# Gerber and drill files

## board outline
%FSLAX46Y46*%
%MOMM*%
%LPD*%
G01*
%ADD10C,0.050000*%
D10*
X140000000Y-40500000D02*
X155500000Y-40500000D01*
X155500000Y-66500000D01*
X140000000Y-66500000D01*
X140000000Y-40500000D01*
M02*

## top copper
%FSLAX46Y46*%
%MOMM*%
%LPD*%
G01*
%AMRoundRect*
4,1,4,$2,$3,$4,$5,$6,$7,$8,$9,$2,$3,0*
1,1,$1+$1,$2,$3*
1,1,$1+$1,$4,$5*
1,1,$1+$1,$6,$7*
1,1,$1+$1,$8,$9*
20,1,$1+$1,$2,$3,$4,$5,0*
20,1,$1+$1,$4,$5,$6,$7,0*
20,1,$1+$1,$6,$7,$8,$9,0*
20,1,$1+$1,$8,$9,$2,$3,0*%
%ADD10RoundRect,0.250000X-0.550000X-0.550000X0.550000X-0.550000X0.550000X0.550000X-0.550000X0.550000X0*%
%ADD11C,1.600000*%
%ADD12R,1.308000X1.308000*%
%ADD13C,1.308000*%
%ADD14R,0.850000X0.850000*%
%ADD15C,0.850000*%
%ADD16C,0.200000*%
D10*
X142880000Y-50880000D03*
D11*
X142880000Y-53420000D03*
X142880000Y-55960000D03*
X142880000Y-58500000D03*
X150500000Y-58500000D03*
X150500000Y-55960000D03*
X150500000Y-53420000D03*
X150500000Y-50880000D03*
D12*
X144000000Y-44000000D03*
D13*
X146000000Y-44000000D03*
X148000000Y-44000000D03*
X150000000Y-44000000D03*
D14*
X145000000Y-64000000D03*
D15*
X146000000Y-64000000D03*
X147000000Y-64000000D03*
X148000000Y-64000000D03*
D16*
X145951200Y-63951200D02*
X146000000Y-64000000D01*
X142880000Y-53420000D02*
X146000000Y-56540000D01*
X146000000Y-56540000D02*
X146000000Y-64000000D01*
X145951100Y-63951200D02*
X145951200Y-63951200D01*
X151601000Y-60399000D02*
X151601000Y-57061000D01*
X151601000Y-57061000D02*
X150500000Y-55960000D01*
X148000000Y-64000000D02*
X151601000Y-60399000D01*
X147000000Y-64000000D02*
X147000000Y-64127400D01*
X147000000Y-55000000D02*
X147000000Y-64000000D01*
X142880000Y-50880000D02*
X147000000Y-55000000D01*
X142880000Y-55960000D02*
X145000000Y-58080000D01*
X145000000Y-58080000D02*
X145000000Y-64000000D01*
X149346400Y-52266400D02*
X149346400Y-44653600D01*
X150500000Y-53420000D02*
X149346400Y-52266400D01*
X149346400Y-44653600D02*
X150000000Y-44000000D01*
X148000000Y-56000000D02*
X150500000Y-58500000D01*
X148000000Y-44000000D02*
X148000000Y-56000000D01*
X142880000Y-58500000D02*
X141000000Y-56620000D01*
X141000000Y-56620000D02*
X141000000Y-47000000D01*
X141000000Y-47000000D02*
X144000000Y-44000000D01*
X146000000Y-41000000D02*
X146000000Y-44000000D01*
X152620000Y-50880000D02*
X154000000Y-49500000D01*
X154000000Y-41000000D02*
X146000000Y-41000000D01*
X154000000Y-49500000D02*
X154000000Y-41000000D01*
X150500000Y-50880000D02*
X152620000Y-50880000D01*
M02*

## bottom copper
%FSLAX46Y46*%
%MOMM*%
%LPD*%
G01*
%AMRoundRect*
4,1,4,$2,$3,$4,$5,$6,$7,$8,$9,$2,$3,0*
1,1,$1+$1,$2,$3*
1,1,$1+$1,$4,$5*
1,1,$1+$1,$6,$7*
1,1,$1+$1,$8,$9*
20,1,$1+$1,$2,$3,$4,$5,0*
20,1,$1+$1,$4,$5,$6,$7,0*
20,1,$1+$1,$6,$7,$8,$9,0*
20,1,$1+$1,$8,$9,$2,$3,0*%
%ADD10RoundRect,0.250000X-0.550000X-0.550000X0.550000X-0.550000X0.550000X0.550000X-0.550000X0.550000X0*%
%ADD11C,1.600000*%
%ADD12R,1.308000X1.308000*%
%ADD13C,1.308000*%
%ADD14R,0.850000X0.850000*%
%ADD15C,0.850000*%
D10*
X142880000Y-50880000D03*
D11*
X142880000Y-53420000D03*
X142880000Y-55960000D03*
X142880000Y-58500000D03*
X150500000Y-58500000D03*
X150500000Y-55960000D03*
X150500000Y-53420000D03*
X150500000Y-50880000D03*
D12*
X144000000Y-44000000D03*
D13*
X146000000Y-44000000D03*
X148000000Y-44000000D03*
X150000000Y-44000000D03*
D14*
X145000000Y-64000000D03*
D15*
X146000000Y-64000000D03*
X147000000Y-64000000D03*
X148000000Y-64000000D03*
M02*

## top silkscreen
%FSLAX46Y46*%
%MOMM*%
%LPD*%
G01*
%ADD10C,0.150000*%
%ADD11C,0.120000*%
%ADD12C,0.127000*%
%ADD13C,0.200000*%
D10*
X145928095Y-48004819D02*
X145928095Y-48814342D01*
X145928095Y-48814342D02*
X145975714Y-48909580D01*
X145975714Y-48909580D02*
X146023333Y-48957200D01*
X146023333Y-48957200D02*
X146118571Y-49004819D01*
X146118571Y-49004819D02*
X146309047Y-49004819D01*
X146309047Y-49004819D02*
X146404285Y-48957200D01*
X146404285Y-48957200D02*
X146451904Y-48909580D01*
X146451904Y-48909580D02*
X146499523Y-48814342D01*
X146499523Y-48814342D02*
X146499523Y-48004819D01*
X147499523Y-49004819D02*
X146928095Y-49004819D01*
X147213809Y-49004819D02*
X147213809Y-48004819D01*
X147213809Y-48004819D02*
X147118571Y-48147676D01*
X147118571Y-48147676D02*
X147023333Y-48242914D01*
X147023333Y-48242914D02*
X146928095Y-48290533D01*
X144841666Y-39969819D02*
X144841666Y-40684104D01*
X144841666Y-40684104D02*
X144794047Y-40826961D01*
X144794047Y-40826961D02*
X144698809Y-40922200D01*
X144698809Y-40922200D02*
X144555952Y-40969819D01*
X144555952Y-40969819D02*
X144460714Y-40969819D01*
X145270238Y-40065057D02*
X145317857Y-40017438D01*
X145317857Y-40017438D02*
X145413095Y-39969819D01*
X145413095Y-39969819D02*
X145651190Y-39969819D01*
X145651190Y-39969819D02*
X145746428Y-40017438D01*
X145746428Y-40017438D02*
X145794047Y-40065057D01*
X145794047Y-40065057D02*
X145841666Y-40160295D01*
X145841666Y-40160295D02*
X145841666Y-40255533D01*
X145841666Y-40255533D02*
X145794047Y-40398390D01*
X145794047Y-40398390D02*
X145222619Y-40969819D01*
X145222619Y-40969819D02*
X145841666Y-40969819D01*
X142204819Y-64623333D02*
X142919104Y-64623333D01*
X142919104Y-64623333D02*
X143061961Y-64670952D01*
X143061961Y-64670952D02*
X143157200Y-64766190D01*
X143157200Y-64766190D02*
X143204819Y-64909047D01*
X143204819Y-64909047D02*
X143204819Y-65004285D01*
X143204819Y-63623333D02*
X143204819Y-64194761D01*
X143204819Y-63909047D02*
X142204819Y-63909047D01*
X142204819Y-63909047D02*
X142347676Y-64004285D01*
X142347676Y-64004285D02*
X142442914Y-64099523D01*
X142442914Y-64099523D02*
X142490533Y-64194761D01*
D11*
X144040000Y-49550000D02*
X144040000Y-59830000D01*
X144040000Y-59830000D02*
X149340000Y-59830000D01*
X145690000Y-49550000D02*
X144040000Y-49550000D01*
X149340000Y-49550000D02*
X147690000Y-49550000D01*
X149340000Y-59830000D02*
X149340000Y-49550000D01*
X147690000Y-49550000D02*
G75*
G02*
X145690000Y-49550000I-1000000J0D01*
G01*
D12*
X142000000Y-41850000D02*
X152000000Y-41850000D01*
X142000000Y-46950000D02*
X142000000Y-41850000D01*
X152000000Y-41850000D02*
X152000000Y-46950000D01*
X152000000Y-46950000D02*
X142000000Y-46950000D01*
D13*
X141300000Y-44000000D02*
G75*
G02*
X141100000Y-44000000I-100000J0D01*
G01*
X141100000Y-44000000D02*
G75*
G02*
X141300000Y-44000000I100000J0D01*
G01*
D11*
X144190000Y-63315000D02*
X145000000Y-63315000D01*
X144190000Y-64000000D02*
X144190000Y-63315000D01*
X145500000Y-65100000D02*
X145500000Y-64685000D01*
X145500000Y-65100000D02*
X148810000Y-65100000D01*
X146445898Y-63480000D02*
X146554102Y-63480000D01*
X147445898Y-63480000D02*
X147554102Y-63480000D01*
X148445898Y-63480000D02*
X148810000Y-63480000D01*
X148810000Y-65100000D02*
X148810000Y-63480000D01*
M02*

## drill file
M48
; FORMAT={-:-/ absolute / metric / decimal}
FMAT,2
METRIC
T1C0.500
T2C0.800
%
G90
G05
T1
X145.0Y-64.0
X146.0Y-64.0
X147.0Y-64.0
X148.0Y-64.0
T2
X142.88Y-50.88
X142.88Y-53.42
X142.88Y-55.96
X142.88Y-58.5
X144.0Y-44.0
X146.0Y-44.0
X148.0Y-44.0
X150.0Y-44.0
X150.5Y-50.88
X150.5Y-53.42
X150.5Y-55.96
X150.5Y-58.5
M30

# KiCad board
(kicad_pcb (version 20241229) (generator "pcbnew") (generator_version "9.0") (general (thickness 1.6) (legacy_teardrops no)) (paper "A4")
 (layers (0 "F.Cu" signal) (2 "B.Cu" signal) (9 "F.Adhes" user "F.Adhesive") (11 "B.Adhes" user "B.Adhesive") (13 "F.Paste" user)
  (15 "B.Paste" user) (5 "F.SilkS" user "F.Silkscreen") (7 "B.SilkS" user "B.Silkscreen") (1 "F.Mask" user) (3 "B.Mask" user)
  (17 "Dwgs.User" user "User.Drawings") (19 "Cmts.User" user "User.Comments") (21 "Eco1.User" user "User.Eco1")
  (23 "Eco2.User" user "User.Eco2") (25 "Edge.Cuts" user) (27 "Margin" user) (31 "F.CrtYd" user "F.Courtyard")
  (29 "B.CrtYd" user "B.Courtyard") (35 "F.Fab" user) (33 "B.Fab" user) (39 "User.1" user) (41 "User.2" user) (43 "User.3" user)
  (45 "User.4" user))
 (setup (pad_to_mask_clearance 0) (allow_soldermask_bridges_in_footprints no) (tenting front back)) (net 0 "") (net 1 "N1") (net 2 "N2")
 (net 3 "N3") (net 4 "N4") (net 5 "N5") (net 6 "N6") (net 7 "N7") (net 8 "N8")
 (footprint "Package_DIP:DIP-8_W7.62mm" (layer "F.Cu") (at 142.88 50.88)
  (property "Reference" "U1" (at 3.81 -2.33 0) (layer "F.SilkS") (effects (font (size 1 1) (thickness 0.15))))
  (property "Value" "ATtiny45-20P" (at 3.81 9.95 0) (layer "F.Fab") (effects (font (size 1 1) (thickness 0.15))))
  (fp_line (start 1.16 -1.33) (end 1.16 8.95) (stroke (width 0.12) (type solid)) (layer "F.SilkS"))
  (fp_line (start 1.16 8.95) (end 6.46 8.95) (stroke (width 0.12) (type solid)) (layer "F.SilkS"))
  (fp_line (start 2.81 -1.33) (end 1.16 -1.33) (stroke (width 0.12) (type solid)) (layer "F.SilkS"))
  (fp_line (start 6.46 -1.33) (end 4.81 -1.33) (stroke (width 0.12) (type solid)) (layer "F.SilkS"))
  (fp_line (start 6.46 8.95) (end 6.46 -1.33) (stroke (width 0.12) (type solid)) (layer "F.SilkS"))
  (fp_arc (start 4.81 -1.33) (mid 3.81 -0.33) (end 2.81 -1.33) (stroke (width 0.12) (type solid)) (layer "F.SilkS"))
  (pad "1" thru_hole roundrect (at 0 0) (size 1.6 1.6) (drill 0.8) (layers "*.Cu" "*.Mask") (remove_unused_layers no)
   (roundrect_rratio 0.15625) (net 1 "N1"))
  (pad "2" thru_hole circle (at 0 2.54) (size 1.6 1.6) (drill 0.8) (layers "*.Cu" "*.Mask") (remove_unused_layers no) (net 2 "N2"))
  (pad "3" thru_hole circle (at 0 5.08) (size 1.6 1.6) (drill 0.8) (layers "*.Cu" "*.Mask") (remove_unused_layers no) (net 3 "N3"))
  (pad "4" thru_hole circle (at 0 7.62) (size 1.6 1.6) (drill 0.8) (layers "*.Cu" "*.Mask") (remove_unused_layers no) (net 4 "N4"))
  (pad "5" thru_hole circle (at 7.62 7.62) (size 1.6 1.6) (drill 0.8) (layers "*.Cu" "*.Mask") (remove_unused_layers no) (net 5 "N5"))
  (pad "6" thru_hole circle (at 7.62 5.08) (size 1.6 1.6) (drill 0.8) (layers "*.Cu" "*.Mask") (remove_unused_layers no) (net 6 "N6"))
  (pad "7" thru_hole circle (at 7.62 2.54) (size 1.6 1.6) (drill 0.8) (layers "*.Cu" "*.Mask") (remove_unused_layers no) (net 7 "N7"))
  (pad "8" thru_hole circle (at 7.62 0) (size 1.6 1.6) (drill 0.8) (layers "*.Cu" "*.Mask") (remove_unused_layers no) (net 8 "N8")))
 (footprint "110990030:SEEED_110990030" (layer "F.Cu") (at 147 44)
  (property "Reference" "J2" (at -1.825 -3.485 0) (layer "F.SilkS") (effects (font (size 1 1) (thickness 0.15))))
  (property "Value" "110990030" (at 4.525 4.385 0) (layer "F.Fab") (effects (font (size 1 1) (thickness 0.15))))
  (fp_line (start -5 -2.15) (end 5 -2.15) (stroke (width 0.127) (type solid)) (layer "F.SilkS"))
  (fp_line (start -5 2.95) (end -5 -2.15) (stroke (width 0.127) (type solid)) (layer "F.SilkS"))
  (fp_line (start 5 -2.15) (end 5 2.95) (stroke (width 0.127) (type solid)) (layer "F.SilkS"))
  (fp_line (start 5 2.95) (end -5 2.95) (stroke (width 0.127) (type solid)) (layer "F.SilkS"))
  (fp_circle (center -5.8 0) (end -5.7 0) (stroke (width 0.2) (type solid)) (fill no) (layer "F.SilkS"))
  (pad "1" thru_hole rect (at -3 0) (size 1.308 1.308) (drill 0.8) (layers "*.Cu" "*.Mask") (remove_unused_layers no) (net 4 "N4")
   (solder_mask_margin 0.102))
  (pad "2" thru_hole circle (at -1 0) (size 1.308 1.308) (drill 0.8) (layers "*.Cu" "*.Mask") (remove_unused_layers no) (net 8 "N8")
   (solder_mask_margin 0.102))
  (pad "3" thru_hole circle (at 1 0) (size 1.308 1.308) (drill 0.8) (layers "*.Cu" "*.Mask") (remove_unused_layers no) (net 5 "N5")
   (solder_mask_margin 0.102))
  (pad "4" thru_hole circle (at 3 0) (size 1.308 1.308) (drill 0.8) (layers "*.Cu" "*.Mask") (remove_unused_layers no) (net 7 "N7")
   (solder_mask_margin 0.102)))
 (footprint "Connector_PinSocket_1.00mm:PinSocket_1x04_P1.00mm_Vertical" (layer "F.Cu") (at 145 64 90)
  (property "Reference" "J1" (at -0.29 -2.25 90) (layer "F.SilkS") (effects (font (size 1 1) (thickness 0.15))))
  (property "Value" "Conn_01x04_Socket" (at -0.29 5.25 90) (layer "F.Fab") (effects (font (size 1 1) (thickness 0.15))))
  (fp_line (start 0.685 -0.81) (end 0.685 0) (stroke (width 0.12) (type solid)) (layer "F.SilkS"))
  (fp_line (start 0 -0.81) (end 0.685 -0.81) (stroke (width 0.12) (type solid)) (layer "F.SilkS"))
  (fp_line (start -1.1 0.5) (end -0.685 0.5) (stroke (width 0.12) (type solid)) (layer "F.SilkS"))
  (fp_line (start -1.1 0.5) (end -1.1 3.81) (stroke (width 0.12) (type solid)) (layer "F.SilkS"))
  (fp_line (start 0.52 1.445898) (end 0.52 1.554102) (stroke (width 0.12) (type solid)) (layer "F.SilkS"))
  (fp_line (start 0.52 2.445898) (end 0.52 2.554102) (stroke (width 0.12) (type solid)) (layer "F.SilkS"))
  (fp_line (start 0.52 3.445898) (end 0.52 3.81) (stroke (width 0.12) (type solid)) (layer "F.SilkS"))
  (fp_line (start -1.1 3.81) (end 0.52 3.81) (stroke (width 0.12) (type solid)) (layer "F.SilkS"))
  (pad "1" thru_hole rect (at 0 0 90) (size 0.85 0.85) (drill 0.5) (layers "*.Cu" "*.Mask") (remove_unused_layers no) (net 3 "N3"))
  (pad "2" thru_hole circle (at 0 1 90) (size 0.85 0.85) (drill 0.5) (layers "*.Cu" "*.Mask") (remove_unused_layers no) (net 2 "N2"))
  (pad "3" thru_hole circle (at 0 2 90) (size 0.85 0.85) (drill 0.5) (layers "*.Cu" "*.Mask") (remove_unused_layers no) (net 1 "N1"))
  (pad "4" thru_hole circle (at 0 3 90) (size 0.85 0.85) (drill 0.5) (layers "*.Cu" "*.Mask") (remove_unused_layers no) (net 6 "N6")))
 (gr_rect (start 140 40.5) (end 155.5 66.5) (stroke (width 0.05) (type default)) (fill no) (layer "Edge.Cuts"))
 (segment (start 145.9512 63.9512) (end 146 64) (width 0.2) (layer "F.Cu") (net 2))
 (segment (start 142.88 53.42) (end 146 56.54) (width 0.2) (layer "F.Cu") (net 2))
 (segment (start 146 56.54) (end 146 64) (width 0.2) (layer "F.Cu") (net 2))
 (segment (start 145.9511 63.9512) (end 145.9512 63.9512) (width 0.2) (layer "F.Cu") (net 2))
 (segment (start 151.601 60.399) (end 151.601 57.061) (width 0.2) (layer "F.Cu") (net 6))
 (segment (start 151.601 57.061) (end 150.5 55.96) (width 0.2) (layer "F.Cu") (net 6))
 (segment (start 148 64) (end 151.601 60.399) (width 0.2) (layer "F.Cu") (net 6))
 (segment (start 147 64) (end 147 64.1274) (width 0.2) (layer "F.Cu") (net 1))
 (segment (start 147 55) (end 147 64) (width 0.2) (layer "F.Cu") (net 1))
 (segment (start 142.88 50.88) (end 147 55) (width 0.2) (layer "F.Cu") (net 1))
 (segment (start 142.88 55.96) (end 145 58.08) (width 0.2) (layer "F.Cu") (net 3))
 (segment (start 145 58.08) (end 145 64) (width 0.2) (layer "F.Cu") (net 3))
 (segment (start 149.3464 52.2664) (end 149.3464 44.6536) (width 0.2) (layer "F.Cu") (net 7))
 (segment (start 150.5 53.42) (end 149.3464 52.2664) (width 0.2) (layer "F.Cu") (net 7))
 (segment (start 149.3464 44.6536) (end 150 44) (width 0.2) (layer "F.Cu") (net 7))
 (segment (start 148 56) (end 150.5 58.5) (width 0.2) (layer "F.Cu") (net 5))
 (segment (start 148 44) (end 148 56) (width 0.2) (layer "F.Cu") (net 5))
 (segment (start 142.88 58.5) (end 141 56.62) (width 0.2) (layer "F.Cu") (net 4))
 (segment (start 141 56.62) (end 141 47) (width 0.2) (layer "F.Cu") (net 4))
 (segment (start 141 47) (end 144 44) (width 0.2) (layer "F.Cu") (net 4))
 (segment (start 146 41) (end 146 44) (width 0.2) (layer "F.Cu") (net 8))
 (segment (start 152.62 50.88) (end 154 49.5) (width 0.2) (layer "F.Cu") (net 8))
 (segment (start 154 41) (end 146 41) (width 0.2) (layer "F.Cu") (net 8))
 (segment (start 154 49.5) (end 154 41) (width 0.2) (layer "F.Cu") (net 8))
 (segment (start 150.5 50.88) (end 152.62 50.88) (width 0.2) (layer "F.Cu") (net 8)))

